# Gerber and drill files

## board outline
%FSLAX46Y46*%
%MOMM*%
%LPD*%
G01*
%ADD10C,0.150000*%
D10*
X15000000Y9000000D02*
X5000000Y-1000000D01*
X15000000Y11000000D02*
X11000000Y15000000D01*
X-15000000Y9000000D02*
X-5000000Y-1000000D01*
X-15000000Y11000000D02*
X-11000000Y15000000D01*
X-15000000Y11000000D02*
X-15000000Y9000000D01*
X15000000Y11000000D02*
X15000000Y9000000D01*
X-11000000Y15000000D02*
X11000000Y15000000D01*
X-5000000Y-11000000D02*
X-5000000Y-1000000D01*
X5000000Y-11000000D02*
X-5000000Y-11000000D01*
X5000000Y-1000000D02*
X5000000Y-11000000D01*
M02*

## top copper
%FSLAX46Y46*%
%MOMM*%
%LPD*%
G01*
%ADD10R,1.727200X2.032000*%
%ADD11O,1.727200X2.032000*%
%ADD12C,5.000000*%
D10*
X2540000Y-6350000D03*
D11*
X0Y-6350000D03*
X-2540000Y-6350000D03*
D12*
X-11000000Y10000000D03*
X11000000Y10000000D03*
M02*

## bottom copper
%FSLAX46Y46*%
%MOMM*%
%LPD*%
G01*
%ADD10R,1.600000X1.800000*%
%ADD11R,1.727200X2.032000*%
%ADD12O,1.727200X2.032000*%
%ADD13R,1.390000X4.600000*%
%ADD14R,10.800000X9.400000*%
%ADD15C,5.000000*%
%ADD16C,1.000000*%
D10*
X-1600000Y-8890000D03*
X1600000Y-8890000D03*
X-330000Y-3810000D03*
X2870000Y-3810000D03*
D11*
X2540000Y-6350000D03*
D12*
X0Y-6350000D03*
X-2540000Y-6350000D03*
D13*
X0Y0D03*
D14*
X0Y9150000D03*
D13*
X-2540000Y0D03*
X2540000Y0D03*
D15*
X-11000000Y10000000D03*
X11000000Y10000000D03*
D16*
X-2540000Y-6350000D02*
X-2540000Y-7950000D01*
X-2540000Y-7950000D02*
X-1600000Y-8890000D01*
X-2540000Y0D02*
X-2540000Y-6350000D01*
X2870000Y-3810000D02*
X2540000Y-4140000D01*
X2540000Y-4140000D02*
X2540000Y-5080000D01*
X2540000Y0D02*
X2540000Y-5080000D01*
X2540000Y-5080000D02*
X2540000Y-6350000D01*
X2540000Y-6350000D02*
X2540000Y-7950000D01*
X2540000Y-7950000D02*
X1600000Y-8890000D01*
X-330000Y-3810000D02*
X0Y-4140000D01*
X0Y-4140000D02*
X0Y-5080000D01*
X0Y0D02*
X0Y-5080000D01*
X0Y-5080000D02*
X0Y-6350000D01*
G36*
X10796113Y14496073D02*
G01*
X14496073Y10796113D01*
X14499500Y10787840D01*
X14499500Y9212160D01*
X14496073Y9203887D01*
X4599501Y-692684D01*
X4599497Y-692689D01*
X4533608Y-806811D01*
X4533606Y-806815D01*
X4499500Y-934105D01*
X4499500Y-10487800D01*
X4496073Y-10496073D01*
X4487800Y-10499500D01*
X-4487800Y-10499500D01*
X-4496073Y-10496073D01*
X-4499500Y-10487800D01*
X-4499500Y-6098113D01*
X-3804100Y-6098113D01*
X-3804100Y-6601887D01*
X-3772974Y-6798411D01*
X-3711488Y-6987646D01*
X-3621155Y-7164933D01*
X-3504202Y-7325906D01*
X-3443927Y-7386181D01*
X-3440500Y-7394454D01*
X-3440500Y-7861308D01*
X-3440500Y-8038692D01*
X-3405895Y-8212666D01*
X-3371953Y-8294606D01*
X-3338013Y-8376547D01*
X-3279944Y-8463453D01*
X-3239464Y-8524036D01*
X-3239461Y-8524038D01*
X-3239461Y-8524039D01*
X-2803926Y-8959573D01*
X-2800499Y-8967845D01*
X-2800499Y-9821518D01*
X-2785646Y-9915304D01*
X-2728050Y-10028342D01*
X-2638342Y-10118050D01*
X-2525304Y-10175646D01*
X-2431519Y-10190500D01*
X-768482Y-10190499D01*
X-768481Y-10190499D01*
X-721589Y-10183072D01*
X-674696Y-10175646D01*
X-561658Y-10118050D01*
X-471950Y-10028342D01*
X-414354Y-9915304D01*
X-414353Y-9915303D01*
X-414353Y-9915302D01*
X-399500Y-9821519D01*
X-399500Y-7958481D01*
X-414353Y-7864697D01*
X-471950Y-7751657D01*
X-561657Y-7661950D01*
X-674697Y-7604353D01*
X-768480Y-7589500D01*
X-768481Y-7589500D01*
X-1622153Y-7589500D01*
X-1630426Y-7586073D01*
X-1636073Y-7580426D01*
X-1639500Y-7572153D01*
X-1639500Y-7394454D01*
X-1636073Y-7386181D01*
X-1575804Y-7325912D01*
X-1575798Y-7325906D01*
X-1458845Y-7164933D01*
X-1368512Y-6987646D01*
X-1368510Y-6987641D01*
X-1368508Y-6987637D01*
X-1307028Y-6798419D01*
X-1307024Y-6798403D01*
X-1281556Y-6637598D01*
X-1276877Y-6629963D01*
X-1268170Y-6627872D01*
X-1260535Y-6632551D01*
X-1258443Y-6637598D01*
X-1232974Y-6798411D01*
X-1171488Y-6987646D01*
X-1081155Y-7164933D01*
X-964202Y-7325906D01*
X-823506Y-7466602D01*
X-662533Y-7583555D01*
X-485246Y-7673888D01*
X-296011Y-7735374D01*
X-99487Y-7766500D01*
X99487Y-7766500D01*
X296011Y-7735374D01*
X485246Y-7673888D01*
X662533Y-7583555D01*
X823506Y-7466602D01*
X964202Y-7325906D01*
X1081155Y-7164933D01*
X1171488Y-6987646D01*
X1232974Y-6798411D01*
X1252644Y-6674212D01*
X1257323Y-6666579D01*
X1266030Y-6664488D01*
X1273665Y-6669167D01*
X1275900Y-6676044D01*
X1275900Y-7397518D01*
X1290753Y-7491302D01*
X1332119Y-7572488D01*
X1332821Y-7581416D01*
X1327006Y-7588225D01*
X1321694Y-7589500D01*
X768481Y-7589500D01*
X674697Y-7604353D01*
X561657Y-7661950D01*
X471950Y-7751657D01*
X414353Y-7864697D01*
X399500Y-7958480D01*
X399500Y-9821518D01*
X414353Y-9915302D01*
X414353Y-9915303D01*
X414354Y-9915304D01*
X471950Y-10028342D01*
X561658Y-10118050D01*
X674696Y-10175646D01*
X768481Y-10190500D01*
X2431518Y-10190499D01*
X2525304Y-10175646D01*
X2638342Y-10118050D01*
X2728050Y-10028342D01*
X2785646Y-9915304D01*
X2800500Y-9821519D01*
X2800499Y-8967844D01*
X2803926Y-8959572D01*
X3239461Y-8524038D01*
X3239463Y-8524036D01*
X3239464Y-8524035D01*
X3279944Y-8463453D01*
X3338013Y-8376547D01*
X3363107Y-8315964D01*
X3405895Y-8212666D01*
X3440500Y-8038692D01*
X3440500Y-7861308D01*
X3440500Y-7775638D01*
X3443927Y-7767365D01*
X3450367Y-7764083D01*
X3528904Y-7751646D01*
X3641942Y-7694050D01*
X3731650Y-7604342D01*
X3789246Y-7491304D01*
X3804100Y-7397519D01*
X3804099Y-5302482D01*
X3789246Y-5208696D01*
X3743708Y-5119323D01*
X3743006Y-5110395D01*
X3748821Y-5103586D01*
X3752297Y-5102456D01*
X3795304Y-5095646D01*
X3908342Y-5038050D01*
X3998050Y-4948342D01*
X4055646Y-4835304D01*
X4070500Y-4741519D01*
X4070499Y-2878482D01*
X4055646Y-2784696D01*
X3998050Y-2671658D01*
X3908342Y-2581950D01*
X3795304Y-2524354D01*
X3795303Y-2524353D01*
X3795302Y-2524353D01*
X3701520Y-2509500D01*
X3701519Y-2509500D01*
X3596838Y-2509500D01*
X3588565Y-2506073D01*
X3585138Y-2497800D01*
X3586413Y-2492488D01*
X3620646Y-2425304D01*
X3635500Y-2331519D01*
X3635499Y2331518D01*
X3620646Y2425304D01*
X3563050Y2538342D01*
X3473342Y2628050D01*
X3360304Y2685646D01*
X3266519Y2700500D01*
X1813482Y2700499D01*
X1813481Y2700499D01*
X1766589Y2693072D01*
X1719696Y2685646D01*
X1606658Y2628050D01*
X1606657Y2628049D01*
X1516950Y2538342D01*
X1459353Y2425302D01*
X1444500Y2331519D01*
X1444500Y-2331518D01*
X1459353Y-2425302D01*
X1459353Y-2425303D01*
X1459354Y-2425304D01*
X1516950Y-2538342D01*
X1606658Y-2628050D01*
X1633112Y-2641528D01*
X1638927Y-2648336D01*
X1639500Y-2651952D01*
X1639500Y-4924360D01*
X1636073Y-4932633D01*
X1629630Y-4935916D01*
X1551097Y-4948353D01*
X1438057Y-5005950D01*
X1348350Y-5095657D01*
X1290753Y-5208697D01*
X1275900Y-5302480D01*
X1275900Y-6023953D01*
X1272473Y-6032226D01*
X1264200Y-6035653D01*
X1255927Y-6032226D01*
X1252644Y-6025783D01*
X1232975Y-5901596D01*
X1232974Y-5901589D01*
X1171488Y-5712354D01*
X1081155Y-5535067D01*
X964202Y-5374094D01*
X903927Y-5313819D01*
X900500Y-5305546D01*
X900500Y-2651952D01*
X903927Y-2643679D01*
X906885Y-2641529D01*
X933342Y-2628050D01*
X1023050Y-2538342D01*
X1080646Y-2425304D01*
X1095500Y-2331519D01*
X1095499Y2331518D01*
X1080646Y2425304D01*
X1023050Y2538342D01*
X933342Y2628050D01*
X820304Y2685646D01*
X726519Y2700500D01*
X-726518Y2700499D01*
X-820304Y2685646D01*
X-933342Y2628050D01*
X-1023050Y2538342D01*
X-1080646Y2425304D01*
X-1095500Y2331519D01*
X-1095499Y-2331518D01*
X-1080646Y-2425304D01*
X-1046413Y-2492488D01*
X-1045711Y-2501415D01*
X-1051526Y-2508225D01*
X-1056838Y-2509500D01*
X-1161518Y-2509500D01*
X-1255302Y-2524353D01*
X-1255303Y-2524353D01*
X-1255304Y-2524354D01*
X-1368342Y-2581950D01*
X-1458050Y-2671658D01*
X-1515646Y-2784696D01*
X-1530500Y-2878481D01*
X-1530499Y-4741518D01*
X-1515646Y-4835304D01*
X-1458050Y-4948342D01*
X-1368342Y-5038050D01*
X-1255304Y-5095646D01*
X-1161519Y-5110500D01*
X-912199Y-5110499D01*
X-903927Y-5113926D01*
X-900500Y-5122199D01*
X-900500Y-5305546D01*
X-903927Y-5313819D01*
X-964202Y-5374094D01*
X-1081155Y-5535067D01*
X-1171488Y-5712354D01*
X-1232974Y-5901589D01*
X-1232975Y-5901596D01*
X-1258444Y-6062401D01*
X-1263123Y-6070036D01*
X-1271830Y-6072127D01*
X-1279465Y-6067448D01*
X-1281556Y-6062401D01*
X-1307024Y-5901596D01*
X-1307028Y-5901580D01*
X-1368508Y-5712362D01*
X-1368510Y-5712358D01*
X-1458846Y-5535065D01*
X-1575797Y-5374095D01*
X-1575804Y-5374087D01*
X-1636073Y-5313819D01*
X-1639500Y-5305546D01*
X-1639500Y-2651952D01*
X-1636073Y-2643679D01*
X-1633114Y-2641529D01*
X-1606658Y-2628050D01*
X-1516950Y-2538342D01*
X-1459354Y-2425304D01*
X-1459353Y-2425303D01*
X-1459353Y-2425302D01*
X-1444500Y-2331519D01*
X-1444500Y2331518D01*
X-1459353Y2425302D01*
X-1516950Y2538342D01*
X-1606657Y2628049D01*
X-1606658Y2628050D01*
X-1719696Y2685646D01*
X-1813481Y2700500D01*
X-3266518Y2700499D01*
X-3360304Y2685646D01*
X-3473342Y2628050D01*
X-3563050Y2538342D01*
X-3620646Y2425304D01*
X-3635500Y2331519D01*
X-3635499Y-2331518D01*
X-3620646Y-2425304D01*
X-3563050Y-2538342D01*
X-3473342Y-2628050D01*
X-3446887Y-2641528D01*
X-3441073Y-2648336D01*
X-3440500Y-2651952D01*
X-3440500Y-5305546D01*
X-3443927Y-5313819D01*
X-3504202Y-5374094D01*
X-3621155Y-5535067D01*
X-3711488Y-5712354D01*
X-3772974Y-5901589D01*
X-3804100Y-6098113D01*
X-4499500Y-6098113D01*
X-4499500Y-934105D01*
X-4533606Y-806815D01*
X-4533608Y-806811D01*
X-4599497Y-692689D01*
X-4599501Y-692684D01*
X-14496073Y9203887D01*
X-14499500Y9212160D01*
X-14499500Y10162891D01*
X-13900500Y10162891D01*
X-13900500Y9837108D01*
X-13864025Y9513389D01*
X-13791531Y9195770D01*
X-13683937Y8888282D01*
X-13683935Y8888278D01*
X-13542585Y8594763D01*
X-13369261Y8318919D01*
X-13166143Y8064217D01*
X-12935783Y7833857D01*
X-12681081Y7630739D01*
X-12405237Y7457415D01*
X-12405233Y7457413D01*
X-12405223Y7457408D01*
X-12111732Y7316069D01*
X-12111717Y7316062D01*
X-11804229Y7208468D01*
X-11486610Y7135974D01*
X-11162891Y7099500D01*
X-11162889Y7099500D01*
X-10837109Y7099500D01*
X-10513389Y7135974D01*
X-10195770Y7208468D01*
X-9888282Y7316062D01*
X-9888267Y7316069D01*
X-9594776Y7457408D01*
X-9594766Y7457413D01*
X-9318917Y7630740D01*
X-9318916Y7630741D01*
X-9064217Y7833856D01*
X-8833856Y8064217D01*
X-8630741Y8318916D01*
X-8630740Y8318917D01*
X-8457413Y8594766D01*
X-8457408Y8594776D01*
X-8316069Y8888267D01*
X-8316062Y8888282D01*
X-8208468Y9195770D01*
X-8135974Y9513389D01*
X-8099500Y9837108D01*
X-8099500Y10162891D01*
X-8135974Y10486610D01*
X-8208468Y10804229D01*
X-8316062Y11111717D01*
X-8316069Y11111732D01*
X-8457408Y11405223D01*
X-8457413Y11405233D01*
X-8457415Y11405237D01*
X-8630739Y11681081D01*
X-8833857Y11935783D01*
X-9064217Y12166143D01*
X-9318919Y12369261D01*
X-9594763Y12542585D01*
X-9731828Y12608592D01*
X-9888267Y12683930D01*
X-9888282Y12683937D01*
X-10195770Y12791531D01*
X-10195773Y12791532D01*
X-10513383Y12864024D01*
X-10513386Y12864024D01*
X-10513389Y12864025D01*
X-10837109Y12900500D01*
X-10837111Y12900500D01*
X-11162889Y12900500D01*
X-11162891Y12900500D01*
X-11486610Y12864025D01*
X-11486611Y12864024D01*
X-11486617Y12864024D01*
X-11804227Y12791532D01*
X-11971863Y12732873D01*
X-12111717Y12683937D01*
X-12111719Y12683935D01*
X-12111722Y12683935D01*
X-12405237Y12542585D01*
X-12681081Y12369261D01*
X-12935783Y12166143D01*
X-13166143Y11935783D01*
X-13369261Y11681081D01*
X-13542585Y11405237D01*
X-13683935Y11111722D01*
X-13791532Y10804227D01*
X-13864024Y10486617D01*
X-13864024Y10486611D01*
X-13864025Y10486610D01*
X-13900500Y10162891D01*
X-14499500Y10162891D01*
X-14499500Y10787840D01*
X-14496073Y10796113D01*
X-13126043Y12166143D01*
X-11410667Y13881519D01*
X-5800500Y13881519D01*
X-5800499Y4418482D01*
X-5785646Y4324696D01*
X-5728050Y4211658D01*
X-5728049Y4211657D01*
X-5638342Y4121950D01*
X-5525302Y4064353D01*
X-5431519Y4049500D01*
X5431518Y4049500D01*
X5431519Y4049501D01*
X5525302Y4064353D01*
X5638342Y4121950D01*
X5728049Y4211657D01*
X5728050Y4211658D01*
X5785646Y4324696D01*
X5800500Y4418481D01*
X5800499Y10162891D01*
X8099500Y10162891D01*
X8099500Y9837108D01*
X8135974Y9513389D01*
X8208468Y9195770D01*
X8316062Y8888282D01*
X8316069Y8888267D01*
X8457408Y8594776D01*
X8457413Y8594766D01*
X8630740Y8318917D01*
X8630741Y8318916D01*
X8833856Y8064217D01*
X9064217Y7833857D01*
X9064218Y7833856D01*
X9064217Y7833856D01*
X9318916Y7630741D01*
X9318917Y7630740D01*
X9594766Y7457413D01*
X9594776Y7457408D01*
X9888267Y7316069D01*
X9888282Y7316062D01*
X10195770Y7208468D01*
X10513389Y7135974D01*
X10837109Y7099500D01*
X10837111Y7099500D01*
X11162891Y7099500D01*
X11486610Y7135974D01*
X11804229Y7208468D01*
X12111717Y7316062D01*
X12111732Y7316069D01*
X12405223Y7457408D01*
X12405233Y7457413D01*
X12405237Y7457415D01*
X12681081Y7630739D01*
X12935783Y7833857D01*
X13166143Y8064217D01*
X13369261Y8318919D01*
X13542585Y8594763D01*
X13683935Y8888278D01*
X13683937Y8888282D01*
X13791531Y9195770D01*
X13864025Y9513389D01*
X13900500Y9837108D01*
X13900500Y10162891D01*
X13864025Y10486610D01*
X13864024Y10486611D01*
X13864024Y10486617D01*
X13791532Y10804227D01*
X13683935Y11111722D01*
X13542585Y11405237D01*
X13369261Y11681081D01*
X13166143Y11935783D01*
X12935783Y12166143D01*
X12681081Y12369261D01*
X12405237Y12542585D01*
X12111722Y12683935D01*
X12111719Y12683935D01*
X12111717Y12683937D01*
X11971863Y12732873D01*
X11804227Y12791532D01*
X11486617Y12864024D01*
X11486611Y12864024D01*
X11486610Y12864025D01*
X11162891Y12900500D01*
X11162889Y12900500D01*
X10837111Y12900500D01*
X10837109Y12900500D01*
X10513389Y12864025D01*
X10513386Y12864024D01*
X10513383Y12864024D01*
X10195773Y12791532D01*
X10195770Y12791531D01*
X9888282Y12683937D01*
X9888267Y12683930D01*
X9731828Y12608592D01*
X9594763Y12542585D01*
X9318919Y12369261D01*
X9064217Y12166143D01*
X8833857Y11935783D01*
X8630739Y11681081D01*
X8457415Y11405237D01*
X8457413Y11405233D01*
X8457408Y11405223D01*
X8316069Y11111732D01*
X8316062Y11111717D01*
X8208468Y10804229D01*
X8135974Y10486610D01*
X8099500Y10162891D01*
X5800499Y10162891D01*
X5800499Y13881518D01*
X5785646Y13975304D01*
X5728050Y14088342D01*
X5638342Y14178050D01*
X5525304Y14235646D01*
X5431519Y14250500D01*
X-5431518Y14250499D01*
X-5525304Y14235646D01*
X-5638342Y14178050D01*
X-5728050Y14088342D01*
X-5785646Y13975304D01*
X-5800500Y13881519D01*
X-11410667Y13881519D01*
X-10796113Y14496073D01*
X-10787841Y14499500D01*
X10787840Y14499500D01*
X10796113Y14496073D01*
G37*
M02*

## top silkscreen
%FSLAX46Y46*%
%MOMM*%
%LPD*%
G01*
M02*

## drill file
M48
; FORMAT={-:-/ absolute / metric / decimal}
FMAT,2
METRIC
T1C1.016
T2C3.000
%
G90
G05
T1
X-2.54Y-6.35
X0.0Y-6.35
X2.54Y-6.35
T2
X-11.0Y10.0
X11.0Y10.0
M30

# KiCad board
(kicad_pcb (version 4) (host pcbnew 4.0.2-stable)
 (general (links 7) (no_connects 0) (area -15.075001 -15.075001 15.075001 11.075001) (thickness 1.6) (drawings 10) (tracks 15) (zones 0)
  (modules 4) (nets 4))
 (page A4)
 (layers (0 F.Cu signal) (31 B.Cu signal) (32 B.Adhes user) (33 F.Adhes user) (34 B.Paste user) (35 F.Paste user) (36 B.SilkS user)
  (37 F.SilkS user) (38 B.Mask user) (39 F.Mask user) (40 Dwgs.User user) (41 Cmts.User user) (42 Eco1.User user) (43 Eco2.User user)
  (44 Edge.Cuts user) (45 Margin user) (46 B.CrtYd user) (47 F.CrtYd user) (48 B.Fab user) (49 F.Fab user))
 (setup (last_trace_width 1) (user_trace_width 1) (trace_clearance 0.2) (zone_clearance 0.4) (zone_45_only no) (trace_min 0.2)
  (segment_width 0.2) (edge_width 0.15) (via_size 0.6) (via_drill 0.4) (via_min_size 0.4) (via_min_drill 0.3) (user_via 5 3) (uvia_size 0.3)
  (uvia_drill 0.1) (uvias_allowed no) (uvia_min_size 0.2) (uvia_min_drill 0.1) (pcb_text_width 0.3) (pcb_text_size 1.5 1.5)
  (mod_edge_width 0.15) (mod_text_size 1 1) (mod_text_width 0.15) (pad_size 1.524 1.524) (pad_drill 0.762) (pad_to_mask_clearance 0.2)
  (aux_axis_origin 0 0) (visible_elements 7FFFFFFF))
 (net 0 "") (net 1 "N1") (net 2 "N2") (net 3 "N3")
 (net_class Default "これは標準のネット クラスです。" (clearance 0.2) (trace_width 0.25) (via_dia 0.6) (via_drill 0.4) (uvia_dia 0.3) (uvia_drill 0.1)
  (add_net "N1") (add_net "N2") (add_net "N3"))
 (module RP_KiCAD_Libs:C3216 (layer B.Cu) (at 0 8.89)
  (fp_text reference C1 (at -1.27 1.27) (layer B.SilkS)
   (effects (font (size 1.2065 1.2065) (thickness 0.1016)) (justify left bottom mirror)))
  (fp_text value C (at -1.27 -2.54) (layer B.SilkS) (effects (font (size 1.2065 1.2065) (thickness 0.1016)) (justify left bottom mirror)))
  (pad 1 smd rect (at -1.6 0) (size 1.6 1.8) (layers B.Cu B.Paste B.Mask) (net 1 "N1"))
  (pad 2 smd rect (at 1.6 0) (size 1.6 1.8) (layers B.Cu B.Paste B.Mask) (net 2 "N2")))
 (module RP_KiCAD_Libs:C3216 (layer B.Cu) (at 1.27 3.81)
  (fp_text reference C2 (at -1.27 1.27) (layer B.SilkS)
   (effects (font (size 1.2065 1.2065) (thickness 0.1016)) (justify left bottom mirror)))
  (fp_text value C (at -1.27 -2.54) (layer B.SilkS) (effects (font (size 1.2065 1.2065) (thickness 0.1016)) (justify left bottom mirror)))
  (pad 1 smd rect (at -1.6 0) (size 1.6 1.8) (layers B.Cu B.Paste B.Mask) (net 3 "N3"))
  (pad 2 smd rect (at 1.6 0) (size 1.6 1.8) (layers B.Cu B.Paste B.Mask) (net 2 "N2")))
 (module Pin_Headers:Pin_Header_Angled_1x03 (layer B.Cu) (at 2.54 6.35 90)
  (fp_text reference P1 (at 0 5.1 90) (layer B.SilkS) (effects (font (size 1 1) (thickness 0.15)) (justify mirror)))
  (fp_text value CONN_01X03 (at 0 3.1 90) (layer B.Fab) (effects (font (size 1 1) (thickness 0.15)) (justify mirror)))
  (pad 1 thru_hole rect (at 0 0 90) (size 2.032 1.7272) (drill 1.016) (layers *.Cu *.Mask B.SilkS) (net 2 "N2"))
  (pad 2 thru_hole oval (at 0 -2.54 90) (size 2.032 1.7272) (drill 1.016) (layers *.Cu *.Mask B.SilkS) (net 3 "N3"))
  (pad 3 thru_hole oval (at 0 -5.08 90) (size 2.032 1.7272) (drill 1.016) (layers *.Cu *.Mask B.SilkS) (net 1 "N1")))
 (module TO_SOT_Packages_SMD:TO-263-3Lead (layer B.Cu) (at 0 0 90)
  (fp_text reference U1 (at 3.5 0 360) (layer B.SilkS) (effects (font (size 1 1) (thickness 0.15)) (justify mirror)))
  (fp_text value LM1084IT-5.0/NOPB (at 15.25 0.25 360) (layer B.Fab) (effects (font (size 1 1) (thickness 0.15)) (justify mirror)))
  (pad 2 smd rect (at 0 0 90) (size 4.6 1.39) (layers B.Cu B.Paste B.Mask) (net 3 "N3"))
  (pad 4 smd rect (at 9.15 0 90) (size 9.4 10.8) (layers B.Cu B.Paste B.Mask))
  (pad 3 smd rect (at 0 -2.54 90) (size 4.6 1.39) (layers B.Cu B.Paste B.Mask) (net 1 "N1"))
  (pad 1 smd rect (at 0 2.54 90) (size 4.6 1.39) (layers B.Cu B.Paste B.Mask) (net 2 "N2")))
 (gr_line (start 15 -9) (end 5 1) (angle 90) (layer Edge.Cuts) (width 0.15))
 (gr_line (start 15 -11) (end 11 -15) (angle 90) (layer Edge.Cuts) (width 0.15))
 (gr_line (start -15 -9) (end -5 1) (angle 90) (layer Edge.Cuts) (width 0.15))
 (gr_line (start -15 -11) (end -11 -15) (angle 90) (layer Edge.Cuts) (width 0.15))
 (gr_line (start -15 -11) (end -15 -9) (angle 90) (layer Edge.Cuts) (width 0.15))
 (gr_line (start 15 -11) (end 15 -9) (angle 90) (layer Edge.Cuts) (width 0.15))
 (gr_line (start -11 -15) (end 11 -15) (angle 90) (layer Edge.Cuts) (width 0.15))
 (gr_line (start -5 11) (end -5 1) (angle 90) (layer Edge.Cuts) (width 0.15))
 (gr_line (start 5 11) (end -5 11) (angle 90) (layer Edge.Cuts) (width 0.15))
 (gr_line (start 5 1) (end 5 11) (angle 90) (layer Edge.Cuts) (width 0.15))
 (via (at -11 -10) (size 5) (drill 3) (layers F.Cu B.Cu) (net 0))
 (via (at 11 -10) (size 5) (drill 3) (layers F.Cu B.Cu) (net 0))
 (segment (start -2.54 6.35) (end -2.54 7.95) (width 1) (layer B.Cu) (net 1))
 (segment (start -2.54 7.95) (end -1.6 8.89) (width 1) (layer B.Cu) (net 1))
 (segment (start -2.54 0) (end -2.54 6.35) (width 1) (layer B.Cu) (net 1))
 (segment (start 2.87 3.81) (end 2.54 4.14) (width 1) (layer B.Cu) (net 2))
 (segment (start 2.54 4.14) (end 2.54 5.08) (width 1) (layer B.Cu) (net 2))
 (segment (start 2.54 0) (end 2.54 5.08) (width 1) (layer B.Cu) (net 2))
 (segment (start 2.54 5.08) (end 2.54 6.35) (width 1) (layer B.Cu) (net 2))
 (segment (start 2.54 6.35) (end 2.54 7.95) (width 1) (layer B.Cu) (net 2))
 (segment (start 2.54 7.95) (end 1.6 8.89) (width 1) (layer B.Cu) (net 2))
 (segment (start -0.33 3.81) (end 0 4.14) (width 1) (layer B.Cu) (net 3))
 (segment (start 0 4.14) (end 0 5.08) (width 1) (layer B.Cu) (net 3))
 (segment (start 0 0) (end 0 5.08) (width 1) (layer B.Cu) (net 3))
 (segment (start 0 5.08) (end 0 6.35) (width 1) (layer B.Cu) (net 3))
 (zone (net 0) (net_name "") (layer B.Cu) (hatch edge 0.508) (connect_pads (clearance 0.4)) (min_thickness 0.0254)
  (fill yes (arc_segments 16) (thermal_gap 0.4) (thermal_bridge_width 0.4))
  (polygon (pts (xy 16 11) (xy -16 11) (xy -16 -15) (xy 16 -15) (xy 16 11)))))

